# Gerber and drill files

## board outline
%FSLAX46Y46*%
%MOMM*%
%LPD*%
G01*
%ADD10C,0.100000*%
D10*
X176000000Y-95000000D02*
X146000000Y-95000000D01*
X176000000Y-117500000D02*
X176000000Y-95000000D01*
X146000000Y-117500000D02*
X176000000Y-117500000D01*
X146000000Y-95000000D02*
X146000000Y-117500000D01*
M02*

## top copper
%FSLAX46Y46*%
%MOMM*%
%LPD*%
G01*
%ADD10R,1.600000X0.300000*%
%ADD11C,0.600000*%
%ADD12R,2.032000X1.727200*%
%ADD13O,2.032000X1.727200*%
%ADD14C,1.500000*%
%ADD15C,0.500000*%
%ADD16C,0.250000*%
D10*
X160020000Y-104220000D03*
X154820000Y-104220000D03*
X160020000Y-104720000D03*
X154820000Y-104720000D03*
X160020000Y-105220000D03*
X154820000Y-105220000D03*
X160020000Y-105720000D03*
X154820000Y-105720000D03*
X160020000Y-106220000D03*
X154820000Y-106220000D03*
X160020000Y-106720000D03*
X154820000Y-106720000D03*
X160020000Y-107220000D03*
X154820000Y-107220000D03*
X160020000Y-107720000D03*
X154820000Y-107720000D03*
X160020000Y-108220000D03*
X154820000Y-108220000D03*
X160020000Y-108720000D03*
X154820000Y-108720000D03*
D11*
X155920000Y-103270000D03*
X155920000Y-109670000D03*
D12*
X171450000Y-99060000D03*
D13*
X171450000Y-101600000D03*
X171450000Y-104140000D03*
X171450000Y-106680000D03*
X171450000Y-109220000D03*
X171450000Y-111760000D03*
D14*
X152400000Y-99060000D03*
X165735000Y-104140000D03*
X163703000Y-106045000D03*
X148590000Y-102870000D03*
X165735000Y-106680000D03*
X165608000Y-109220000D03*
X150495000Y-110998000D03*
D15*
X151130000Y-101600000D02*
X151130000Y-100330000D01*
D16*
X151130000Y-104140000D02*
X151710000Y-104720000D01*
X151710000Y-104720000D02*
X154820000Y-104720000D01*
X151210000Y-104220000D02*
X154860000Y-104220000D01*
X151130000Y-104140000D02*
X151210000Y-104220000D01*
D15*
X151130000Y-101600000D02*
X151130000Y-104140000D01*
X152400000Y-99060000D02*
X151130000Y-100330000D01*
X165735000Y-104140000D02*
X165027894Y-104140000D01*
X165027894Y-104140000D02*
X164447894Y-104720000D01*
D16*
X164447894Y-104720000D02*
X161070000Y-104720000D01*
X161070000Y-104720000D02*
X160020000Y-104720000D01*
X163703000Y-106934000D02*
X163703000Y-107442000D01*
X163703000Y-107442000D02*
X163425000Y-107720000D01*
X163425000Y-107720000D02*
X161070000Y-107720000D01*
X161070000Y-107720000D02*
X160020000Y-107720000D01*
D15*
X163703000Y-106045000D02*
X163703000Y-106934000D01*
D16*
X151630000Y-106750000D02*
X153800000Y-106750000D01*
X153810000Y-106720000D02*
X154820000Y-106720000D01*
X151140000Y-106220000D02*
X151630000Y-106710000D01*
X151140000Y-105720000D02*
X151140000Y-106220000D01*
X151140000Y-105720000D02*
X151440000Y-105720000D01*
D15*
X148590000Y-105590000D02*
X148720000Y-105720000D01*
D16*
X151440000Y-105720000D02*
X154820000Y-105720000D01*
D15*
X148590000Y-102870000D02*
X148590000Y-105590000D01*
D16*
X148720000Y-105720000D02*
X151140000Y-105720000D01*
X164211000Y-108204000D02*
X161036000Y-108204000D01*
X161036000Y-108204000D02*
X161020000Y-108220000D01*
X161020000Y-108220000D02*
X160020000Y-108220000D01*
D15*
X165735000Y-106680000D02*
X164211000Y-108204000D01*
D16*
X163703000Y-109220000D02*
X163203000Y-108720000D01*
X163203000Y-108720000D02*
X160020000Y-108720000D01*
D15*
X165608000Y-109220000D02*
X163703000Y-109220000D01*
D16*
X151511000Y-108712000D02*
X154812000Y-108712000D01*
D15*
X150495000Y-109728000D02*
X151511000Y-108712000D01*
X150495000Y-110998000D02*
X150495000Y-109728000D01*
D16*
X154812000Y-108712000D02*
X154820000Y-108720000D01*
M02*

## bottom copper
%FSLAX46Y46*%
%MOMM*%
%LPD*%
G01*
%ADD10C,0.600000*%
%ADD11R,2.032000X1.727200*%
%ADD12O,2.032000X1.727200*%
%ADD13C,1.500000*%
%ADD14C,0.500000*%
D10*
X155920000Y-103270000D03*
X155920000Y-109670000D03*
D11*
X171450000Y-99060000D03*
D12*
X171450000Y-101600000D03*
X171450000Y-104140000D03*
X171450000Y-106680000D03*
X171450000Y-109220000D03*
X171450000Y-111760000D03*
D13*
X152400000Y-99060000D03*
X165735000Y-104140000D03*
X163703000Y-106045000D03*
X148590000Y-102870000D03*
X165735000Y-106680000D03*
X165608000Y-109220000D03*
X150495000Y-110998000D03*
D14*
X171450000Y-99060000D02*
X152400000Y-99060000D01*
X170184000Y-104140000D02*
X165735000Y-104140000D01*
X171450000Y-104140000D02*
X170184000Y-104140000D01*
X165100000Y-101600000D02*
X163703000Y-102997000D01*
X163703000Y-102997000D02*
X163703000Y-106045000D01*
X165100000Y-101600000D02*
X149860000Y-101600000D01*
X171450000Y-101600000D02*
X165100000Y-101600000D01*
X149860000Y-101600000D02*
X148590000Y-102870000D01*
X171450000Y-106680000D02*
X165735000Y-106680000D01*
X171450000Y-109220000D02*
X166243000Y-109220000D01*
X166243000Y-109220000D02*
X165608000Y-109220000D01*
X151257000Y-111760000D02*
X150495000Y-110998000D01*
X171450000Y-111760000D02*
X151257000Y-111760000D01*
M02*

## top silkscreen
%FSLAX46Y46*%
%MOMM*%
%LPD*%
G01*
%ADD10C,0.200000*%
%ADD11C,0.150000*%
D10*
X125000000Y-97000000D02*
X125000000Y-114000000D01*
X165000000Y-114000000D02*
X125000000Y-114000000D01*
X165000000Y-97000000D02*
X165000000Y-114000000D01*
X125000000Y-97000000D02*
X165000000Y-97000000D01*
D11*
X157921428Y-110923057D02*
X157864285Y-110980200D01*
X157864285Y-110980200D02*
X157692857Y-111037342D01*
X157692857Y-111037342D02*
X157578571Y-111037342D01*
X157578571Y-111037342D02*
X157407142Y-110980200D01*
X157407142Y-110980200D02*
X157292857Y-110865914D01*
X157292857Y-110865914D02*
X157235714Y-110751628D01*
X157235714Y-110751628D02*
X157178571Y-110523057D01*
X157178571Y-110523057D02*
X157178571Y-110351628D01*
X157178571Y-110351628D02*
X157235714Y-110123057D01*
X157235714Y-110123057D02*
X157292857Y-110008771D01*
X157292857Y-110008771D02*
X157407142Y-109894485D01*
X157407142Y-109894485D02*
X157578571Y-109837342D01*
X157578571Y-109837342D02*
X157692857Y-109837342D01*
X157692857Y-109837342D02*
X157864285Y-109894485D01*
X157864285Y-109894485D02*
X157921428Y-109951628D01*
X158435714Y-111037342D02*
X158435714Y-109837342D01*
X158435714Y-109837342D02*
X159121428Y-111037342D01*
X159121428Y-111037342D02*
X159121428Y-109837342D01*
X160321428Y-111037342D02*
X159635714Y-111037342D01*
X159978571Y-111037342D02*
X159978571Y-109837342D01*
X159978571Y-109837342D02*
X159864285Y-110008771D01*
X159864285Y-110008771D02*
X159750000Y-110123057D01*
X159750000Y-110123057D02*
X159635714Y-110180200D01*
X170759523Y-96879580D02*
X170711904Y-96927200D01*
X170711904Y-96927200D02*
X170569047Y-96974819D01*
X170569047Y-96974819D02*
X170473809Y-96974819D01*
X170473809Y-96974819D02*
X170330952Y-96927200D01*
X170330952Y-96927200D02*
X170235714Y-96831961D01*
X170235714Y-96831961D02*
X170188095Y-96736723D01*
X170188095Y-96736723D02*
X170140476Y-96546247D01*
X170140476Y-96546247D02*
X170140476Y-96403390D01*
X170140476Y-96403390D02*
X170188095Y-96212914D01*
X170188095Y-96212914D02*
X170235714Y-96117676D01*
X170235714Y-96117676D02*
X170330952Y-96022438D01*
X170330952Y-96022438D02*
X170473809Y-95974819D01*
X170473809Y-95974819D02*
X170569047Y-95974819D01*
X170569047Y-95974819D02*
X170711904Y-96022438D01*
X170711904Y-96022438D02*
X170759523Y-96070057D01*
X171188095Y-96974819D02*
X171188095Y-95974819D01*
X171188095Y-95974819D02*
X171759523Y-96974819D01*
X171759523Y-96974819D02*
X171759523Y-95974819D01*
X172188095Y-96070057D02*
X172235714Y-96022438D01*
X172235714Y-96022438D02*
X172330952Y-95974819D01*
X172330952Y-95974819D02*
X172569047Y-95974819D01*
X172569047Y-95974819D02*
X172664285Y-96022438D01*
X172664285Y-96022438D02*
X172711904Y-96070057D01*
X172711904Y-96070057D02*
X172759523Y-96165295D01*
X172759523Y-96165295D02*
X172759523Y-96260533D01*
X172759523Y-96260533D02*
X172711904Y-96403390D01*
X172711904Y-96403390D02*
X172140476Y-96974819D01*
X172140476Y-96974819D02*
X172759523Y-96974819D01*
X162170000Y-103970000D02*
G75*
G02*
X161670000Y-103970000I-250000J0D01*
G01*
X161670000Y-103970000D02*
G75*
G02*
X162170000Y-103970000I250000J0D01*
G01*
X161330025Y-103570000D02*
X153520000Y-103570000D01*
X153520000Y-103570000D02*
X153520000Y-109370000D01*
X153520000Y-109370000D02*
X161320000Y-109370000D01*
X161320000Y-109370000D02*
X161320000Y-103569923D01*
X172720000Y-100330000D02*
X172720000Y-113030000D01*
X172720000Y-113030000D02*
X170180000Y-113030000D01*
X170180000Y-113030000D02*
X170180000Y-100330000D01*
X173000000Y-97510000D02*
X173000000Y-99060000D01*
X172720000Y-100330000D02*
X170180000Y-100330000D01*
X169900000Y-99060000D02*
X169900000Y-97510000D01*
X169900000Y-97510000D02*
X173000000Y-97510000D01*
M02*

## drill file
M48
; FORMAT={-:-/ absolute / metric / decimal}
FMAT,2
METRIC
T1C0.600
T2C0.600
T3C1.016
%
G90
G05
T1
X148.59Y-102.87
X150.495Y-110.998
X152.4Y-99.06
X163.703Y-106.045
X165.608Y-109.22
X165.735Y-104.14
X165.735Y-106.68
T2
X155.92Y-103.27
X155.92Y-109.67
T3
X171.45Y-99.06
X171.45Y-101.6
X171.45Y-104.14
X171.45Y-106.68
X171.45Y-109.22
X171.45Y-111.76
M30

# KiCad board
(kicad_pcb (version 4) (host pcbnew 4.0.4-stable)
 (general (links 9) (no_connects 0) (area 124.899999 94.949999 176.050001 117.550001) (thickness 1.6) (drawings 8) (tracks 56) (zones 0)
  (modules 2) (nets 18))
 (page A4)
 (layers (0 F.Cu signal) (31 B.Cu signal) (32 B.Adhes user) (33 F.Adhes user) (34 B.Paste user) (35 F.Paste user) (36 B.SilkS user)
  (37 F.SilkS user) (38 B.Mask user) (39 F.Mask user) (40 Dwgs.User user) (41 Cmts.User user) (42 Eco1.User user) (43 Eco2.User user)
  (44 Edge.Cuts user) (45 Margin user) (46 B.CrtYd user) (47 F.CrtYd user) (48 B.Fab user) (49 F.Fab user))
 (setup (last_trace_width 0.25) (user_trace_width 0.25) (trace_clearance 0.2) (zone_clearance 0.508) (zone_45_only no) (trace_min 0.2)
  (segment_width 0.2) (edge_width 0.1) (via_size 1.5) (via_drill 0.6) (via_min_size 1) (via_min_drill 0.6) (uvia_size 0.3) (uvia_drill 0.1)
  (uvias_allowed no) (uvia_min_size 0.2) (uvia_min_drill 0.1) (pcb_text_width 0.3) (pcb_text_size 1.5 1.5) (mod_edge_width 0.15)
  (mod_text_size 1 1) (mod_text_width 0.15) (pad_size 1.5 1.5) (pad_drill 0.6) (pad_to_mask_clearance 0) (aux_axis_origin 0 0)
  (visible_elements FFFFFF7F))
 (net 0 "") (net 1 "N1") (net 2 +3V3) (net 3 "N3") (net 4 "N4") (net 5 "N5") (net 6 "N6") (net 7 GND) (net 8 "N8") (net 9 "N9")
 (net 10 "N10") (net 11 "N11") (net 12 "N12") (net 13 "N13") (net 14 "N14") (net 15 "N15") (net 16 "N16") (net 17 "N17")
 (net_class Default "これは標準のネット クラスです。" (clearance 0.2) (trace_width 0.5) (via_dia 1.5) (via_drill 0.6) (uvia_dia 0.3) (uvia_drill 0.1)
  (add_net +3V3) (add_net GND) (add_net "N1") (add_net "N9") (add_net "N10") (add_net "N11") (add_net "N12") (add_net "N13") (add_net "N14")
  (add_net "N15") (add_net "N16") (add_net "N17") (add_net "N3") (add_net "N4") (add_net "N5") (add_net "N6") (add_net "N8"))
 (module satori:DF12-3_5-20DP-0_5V (layer F.Cu) (at 157.42 106.47 270)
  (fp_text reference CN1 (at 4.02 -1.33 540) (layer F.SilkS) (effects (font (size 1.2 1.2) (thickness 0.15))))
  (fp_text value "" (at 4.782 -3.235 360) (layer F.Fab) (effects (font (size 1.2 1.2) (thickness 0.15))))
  (fp_circle (center -2.5 -4.5) (end -2.25 -4.5) (layer F.SilkS) (width 0.15))
  (fp_line (start -2.9 -3.910025) (end -2.9 3.9) (layer F.SilkS) (width 0.15))
  (fp_line (start -2.9 3.9) (end 2.9 3.9) (layer F.SilkS) (width 0.15))
  (fp_line (start 2.9 3.9) (end 2.9 -3.9) (layer F.SilkS) (width 0.15))
  (fp_line (start 2.9 -3.9) (end -2.900077 -3.9) (layer F.SilkS) (width 0.15))
  (pad 1 smd rect (at -2.25 -2.6 270) (size 0.3 1.6) (layers F.Cu F.Paste F.Mask) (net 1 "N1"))
  (pad 2 smd rect (at -2.25 2.6 270) (size 0.3 1.6) (layers F.Cu F.Paste F.Mask) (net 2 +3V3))
  (pad 3 smd rect (at -1.75 -2.6 270) (size 0.3 1.6) (layers F.Cu F.Paste F.Mask) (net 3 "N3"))
  (pad 4 smd rect (at -1.75 2.6 270) (size 0.3 1.6) (layers F.Cu F.Paste F.Mask) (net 2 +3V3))
  (pad 5 smd rect (at -1.25 -2.6 270) (size 0.3 1.6) (layers F.Cu F.Paste F.Mask) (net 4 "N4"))
  (pad 6 smd rect (at -1.25 2.6 270) (size 0.3 1.6) (layers F.Cu F.Paste F.Mask) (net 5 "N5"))
  (pad 7 smd rect (at -0.75 -2.6 270) (size 0.3 1.6) (layers F.Cu F.Paste F.Mask) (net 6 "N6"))
  (pad 8 smd rect (at -0.75 2.6 270) (size 0.3 1.6) (layers F.Cu F.Paste F.Mask) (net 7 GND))
  (pad 9 smd rect (at -0.25 -2.6 270) (size 0.3 1.6) (layers F.Cu F.Paste F.Mask) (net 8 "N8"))
  (pad 10 smd rect (at -0.25 2.6 270) (size 0.3 1.6) (layers F.Cu F.Paste F.Mask) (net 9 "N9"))
  (pad 11 smd rect (at 0.25 -2.6 270) (size 0.3 1.6) (layers F.Cu F.Paste F.Mask) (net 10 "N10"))
  (pad 12 smd rect (at 0.25 2.6 270) (size 0.3 1.6) (layers F.Cu F.Paste F.Mask) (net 7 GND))
  (pad 13 smd rect (at 0.75 -2.6 270) (size 0.3 1.6) (layers F.Cu F.Paste F.Mask) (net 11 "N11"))
  (pad 14 smd rect (at 0.75 2.6 270) (size 0.3 1.6) (layers F.Cu F.Paste F.Mask) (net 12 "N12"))
  (pad 15 smd rect (at 1.25 -2.6 270) (size 0.3 1.6) (layers F.Cu F.Paste F.Mask) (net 7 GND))
  (pad 16 smd rect (at 1.25 2.6 270) (size 0.3 1.6) (layers F.Cu F.Paste F.Mask) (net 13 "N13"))
  (pad 17 smd rect (at 1.75 -2.6 270) (size 0.3 1.6) (layers F.Cu F.Paste F.Mask) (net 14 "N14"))
  (pad 18 smd rect (at 1.75 2.6 270) (size 0.3 1.6) (layers F.Cu F.Paste F.Mask) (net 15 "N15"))
  (pad 19 smd rect (at 2.25 -2.6 270) (size 0.3 1.6) (layers F.Cu F.Paste F.Mask) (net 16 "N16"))
  (pad 20 smd rect (at 2.25 2.6 270) (size 0.3 1.6) (layers F.Cu F.Paste F.Mask) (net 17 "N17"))
  (pad 21 thru_hole circle (at -3.2 1.5 270) (size 0.6 0.6) (drill 0.6) (layers *.Cu *.Mask) (zone_connect 0))
  (pad 22 thru_hole circle (at 3.2 1.5 270) (size 0.6 0.6) (drill 0.6) (layers *.Cu *.Mask) (zone_connect 0)))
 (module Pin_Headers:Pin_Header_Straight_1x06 (layer F.Cu) (at 171.45 99.06)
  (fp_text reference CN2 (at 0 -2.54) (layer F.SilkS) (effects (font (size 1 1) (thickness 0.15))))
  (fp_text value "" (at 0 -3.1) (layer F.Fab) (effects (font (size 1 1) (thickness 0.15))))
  (fp_line (start 1.27 1.27) (end 1.27 13.97) (layer F.SilkS) (width 0.15))
  (fp_line (start 1.27 13.97) (end -1.27 13.97) (layer F.SilkS) (width 0.15))
  (fp_line (start -1.27 13.97) (end -1.27 1.27) (layer F.SilkS) (width 0.15))
  (fp_line (start 1.55 -1.55) (end 1.55 0) (layer F.SilkS) (width 0.15))
  (fp_line (start 1.27 1.27) (end -1.27 1.27) (layer F.SilkS) (width 0.15))
  (fp_line (start -1.55 0) (end -1.55 -1.55) (layer F.SilkS) (width 0.15))
  (fp_line (start -1.55 -1.55) (end 1.55 -1.55) (layer F.SilkS) (width 0.15))
  (pad 1 thru_hole rect (at 0 0) (size 2.032 1.7272) (drill 1.016) (layers *.Cu *.Mask) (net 2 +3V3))
  (pad 2 thru_hole oval (at 0 2.54) (size 2.032 1.7272) (drill 1.016) (layers *.Cu *.Mask) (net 7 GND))
  (pad 3 thru_hole oval (at 0 5.08) (size 2.032 1.7272) (drill 1.016) (layers *.Cu *.Mask) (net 3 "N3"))
  (pad 4 thru_hole oval (at 0 7.62) (size 2.032 1.7272) (drill 1.016) (layers *.Cu *.Mask) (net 14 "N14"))
  (pad 5 thru_hole oval (at 0 10.16) (size 2.032 1.7272) (drill 1.016) (layers *.Cu *.Mask) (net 16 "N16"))
  (pad 6 thru_hole oval (at 0 12.7) (size 2.032 1.7272) (drill 1.016) (layers *.Cu *.Mask) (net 17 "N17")))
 (gr_line (start 176 95) (end 146 95) (angle 90) (layer Edge.Cuts) (width 0.1))
 (gr_line (start 176 117.5) (end 176 95) (angle 90) (layer Edge.Cuts) (width 0.1))
 (gr_line (start 146 117.5) (end 176 117.5) (angle 90) (layer Edge.Cuts) (width 0.1))
 (gr_line (start 146 95) (end 146 117.5) (angle 90) (layer Edge.Cuts) (width 0.1))
 (gr_line (start 125 97) (end 125 114) (layer F.SilkS) (width 0.2))
 (gr_line (start 165 114) (end 125 114) (layer F.SilkS) (width 0.2))
 (gr_line (start 165 97) (end 165 114) (layer F.SilkS) (width 0.2))
 (gr_line (start 125 97) (end 165 97) (layer F.SilkS) (width 0.2))
 (segment (start 151.13 101.6) (end 151.13 100.33) (width 0.5) (layer F.Cu) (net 2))
 (segment (start 151.13 104.14) (end 151.71 104.72) (width 0.25) (layer F.Cu) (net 2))
 (segment (start 151.71 104.72) (end 154.82 104.72) (width 0.25) (layer F.Cu) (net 2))
 (segment (start 171.45 99.06) (end 152.4 99.06) (width 0.5) (layer B.Cu) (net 2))
 (segment (start 151.21 104.22) (end 154.86 104.22) (width 0.25) (layer F.Cu) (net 2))
 (segment (start 151.13 104.14) (end 151.21 104.22) (width 0.25) (layer F.Cu) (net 2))
 (segment (start 151.13 101.6) (end 151.13 104.14) (width 0.5) (layer F.Cu) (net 2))
 (segment (start 152.4 99.06) (end 151.13 100.33) (width 0.5) (layer F.Cu) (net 2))
 (via (at 152.4 99.06) (size 1.5) (drill 0.6) (layers F.Cu B.Cu) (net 2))
 (segment (start 165.735 104.14) (end 165.027894 104.14) (width 0.5) (layer F.Cu) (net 3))
 (segment (start 165.027894 104.14) (end 164.447894 104.72) (width 0.5) (layer F.Cu) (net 3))
 (segment (start 164.447894 104.72) (end 161.07 104.72) (width 0.25) (layer F.Cu) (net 3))
 (segment (start 161.07 104.72) (end 160.02 104.72) (width 0.25) (layer F.Cu) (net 3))
 (via (at 165.735 104.14) (size 1.5) (drill 0.6) (layers F.Cu B.Cu) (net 3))
 (segment (start 170.184 104.14) (end 165.735 104.14) (width 0.5) (layer B.Cu) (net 3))
 (segment (start 171.45 104.14) (end 170.184 104.14) (width 0.5) (layer B.Cu) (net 3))
 (segment (start 163.703 106.934) (end 163.703 107.442) (width 0.25) (layer F.Cu) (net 7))
 (segment (start 163.703 107.442) (end 163.425 107.72) (width 0.25) (layer F.Cu) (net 7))
 (segment (start 163.425 107.72) (end 161.07 107.72) (width 0.25) (layer F.Cu) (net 7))
 (segment (start 161.07 107.72) (end 160.02 107.72) (width 0.25) (layer F.Cu) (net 7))
 (segment (start 163.703 106.045) (end 163.703 106.934) (width 0.5) (layer F.Cu) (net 7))
 (segment (start 165.1 101.6) (end 163.703 102.997) (width 0.5) (layer B.Cu) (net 7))
 (segment (start 163.703 102.997) (end 163.703 106.045) (width 0.5) (layer B.Cu) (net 7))
 (via (at 163.703 106.045) (size 1.5) (drill 0.6) (layers F.Cu B.Cu) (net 7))
 (segment (start 165.1 101.6) (end 149.86 101.6) (width 0.5) (layer B.Cu) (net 7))
 (segment (start 171.45 101.6) (end 165.1 101.6) (width 0.5) (layer B.Cu) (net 7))
 (segment (start 151.63 106.75) (end 153.8 106.75) (width 0.25) (layer F.Cu) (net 7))
 (segment (start 153.81 106.72) (end 154.82 106.72) (width 0.25) (layer F.Cu) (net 7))
 (segment (start 151.14 106.22) (end 151.63 106.71) (width 0.25) (layer F.Cu) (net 7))
 (segment (start 151.14 105.72) (end 151.14 106.22) (width 0.25) (layer F.Cu) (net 7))
 (segment (start 151.14 105.72) (end 151.44 105.72) (width 0.25) (layer F.Cu) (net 7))
 (segment (start 148.59 105.59) (end 148.72 105.72) (width 0.5) (layer F.Cu) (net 7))
 (segment (start 151.44 105.72) (end 154.82 105.72) (width 0.25) (layer F.Cu) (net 7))
 (via (at 148.59 102.87) (size 1.5) (drill 0.6) (layers F.Cu B.Cu) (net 7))
 (segment (start 149.86 101.6) (end 148.59 102.87) (width 0.5) (layer B.Cu) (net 7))
 (segment (start 148.59 102.87) (end 148.59 105.59) (width 0.5) (layer F.Cu) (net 7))
 (segment (start 148.72 105.72) (end 151.14 105.72) (width 0.25) (layer F.Cu) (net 7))
 (segment (start 164.211 108.204) (end 161.036 108.204) (width 0.25) (layer F.Cu) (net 14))
 (segment (start 161.036 108.204) (end 161.02 108.22) (width 0.25) (layer F.Cu) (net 14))
 (segment (start 161.02 108.22) (end 160.02 108.22) (width 0.25) (layer F.Cu) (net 14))
 (segment (start 171.45 106.68) (end 165.735 106.68) (width 0.5) (layer B.Cu) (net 14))
 (segment (start 165.735 106.68) (end 164.211 108.204) (width 0.5) (layer F.Cu) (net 14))
 (via (at 165.735 106.68) (size 1.5) (drill 0.6) (layers F.Cu B.Cu) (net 14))
 (segment (start 163.703 109.22) (end 163.203 108.72) (width 0.25) (layer F.Cu) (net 16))
 (segment (start 163.203 108.72) (end 160.02 108.72) (width 0.25) (layer F.Cu) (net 16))
 (via (at 165.608 109.22) (size 1.5) (drill 0.6) (layers F.Cu B.Cu) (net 16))
 (segment (start 171.45 109.22) (end 166.243 109.22) (width 0.5) (layer B.Cu) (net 16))
 (segment (start 166.243 109.22) (end 165.608 109.22) (width 0.5) (layer B.Cu) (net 16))
 (segment (start 165.608 109.22) (end 163.703 109.22) (width 0.5) (layer F.Cu) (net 16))
 (via (at 150.495 110.998) (size 1.5) (drill 0.6) (layers F.Cu B.Cu) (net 17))
 (segment (start 151.257 111.76) (end 150.495 110.998) (width 0.5) (layer B.Cu) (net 17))
 (segment (start 171.45 111.76) (end 151.257 111.76) (width 0.5) (layer B.Cu) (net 17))
 (segment (start 151.511 108.712) (end 154.812 108.712) (width 0.25) (layer F.Cu) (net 17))
 (segment (start 150.495 109.728) (end 151.511 108.712) (width 0.5) (layer F.Cu) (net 17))
 (segment (start 150.495 110.998) (end 150.495 109.728) (width 0.5) (layer F.Cu) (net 17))
 (segment (start 154.812 108.712) (end 154.82 108.72) (width 0.25) (layer F.Cu) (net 17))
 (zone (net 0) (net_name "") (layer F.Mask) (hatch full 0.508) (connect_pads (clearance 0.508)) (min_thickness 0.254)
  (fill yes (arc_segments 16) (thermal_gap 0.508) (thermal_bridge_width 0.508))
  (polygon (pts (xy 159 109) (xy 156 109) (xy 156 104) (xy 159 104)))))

